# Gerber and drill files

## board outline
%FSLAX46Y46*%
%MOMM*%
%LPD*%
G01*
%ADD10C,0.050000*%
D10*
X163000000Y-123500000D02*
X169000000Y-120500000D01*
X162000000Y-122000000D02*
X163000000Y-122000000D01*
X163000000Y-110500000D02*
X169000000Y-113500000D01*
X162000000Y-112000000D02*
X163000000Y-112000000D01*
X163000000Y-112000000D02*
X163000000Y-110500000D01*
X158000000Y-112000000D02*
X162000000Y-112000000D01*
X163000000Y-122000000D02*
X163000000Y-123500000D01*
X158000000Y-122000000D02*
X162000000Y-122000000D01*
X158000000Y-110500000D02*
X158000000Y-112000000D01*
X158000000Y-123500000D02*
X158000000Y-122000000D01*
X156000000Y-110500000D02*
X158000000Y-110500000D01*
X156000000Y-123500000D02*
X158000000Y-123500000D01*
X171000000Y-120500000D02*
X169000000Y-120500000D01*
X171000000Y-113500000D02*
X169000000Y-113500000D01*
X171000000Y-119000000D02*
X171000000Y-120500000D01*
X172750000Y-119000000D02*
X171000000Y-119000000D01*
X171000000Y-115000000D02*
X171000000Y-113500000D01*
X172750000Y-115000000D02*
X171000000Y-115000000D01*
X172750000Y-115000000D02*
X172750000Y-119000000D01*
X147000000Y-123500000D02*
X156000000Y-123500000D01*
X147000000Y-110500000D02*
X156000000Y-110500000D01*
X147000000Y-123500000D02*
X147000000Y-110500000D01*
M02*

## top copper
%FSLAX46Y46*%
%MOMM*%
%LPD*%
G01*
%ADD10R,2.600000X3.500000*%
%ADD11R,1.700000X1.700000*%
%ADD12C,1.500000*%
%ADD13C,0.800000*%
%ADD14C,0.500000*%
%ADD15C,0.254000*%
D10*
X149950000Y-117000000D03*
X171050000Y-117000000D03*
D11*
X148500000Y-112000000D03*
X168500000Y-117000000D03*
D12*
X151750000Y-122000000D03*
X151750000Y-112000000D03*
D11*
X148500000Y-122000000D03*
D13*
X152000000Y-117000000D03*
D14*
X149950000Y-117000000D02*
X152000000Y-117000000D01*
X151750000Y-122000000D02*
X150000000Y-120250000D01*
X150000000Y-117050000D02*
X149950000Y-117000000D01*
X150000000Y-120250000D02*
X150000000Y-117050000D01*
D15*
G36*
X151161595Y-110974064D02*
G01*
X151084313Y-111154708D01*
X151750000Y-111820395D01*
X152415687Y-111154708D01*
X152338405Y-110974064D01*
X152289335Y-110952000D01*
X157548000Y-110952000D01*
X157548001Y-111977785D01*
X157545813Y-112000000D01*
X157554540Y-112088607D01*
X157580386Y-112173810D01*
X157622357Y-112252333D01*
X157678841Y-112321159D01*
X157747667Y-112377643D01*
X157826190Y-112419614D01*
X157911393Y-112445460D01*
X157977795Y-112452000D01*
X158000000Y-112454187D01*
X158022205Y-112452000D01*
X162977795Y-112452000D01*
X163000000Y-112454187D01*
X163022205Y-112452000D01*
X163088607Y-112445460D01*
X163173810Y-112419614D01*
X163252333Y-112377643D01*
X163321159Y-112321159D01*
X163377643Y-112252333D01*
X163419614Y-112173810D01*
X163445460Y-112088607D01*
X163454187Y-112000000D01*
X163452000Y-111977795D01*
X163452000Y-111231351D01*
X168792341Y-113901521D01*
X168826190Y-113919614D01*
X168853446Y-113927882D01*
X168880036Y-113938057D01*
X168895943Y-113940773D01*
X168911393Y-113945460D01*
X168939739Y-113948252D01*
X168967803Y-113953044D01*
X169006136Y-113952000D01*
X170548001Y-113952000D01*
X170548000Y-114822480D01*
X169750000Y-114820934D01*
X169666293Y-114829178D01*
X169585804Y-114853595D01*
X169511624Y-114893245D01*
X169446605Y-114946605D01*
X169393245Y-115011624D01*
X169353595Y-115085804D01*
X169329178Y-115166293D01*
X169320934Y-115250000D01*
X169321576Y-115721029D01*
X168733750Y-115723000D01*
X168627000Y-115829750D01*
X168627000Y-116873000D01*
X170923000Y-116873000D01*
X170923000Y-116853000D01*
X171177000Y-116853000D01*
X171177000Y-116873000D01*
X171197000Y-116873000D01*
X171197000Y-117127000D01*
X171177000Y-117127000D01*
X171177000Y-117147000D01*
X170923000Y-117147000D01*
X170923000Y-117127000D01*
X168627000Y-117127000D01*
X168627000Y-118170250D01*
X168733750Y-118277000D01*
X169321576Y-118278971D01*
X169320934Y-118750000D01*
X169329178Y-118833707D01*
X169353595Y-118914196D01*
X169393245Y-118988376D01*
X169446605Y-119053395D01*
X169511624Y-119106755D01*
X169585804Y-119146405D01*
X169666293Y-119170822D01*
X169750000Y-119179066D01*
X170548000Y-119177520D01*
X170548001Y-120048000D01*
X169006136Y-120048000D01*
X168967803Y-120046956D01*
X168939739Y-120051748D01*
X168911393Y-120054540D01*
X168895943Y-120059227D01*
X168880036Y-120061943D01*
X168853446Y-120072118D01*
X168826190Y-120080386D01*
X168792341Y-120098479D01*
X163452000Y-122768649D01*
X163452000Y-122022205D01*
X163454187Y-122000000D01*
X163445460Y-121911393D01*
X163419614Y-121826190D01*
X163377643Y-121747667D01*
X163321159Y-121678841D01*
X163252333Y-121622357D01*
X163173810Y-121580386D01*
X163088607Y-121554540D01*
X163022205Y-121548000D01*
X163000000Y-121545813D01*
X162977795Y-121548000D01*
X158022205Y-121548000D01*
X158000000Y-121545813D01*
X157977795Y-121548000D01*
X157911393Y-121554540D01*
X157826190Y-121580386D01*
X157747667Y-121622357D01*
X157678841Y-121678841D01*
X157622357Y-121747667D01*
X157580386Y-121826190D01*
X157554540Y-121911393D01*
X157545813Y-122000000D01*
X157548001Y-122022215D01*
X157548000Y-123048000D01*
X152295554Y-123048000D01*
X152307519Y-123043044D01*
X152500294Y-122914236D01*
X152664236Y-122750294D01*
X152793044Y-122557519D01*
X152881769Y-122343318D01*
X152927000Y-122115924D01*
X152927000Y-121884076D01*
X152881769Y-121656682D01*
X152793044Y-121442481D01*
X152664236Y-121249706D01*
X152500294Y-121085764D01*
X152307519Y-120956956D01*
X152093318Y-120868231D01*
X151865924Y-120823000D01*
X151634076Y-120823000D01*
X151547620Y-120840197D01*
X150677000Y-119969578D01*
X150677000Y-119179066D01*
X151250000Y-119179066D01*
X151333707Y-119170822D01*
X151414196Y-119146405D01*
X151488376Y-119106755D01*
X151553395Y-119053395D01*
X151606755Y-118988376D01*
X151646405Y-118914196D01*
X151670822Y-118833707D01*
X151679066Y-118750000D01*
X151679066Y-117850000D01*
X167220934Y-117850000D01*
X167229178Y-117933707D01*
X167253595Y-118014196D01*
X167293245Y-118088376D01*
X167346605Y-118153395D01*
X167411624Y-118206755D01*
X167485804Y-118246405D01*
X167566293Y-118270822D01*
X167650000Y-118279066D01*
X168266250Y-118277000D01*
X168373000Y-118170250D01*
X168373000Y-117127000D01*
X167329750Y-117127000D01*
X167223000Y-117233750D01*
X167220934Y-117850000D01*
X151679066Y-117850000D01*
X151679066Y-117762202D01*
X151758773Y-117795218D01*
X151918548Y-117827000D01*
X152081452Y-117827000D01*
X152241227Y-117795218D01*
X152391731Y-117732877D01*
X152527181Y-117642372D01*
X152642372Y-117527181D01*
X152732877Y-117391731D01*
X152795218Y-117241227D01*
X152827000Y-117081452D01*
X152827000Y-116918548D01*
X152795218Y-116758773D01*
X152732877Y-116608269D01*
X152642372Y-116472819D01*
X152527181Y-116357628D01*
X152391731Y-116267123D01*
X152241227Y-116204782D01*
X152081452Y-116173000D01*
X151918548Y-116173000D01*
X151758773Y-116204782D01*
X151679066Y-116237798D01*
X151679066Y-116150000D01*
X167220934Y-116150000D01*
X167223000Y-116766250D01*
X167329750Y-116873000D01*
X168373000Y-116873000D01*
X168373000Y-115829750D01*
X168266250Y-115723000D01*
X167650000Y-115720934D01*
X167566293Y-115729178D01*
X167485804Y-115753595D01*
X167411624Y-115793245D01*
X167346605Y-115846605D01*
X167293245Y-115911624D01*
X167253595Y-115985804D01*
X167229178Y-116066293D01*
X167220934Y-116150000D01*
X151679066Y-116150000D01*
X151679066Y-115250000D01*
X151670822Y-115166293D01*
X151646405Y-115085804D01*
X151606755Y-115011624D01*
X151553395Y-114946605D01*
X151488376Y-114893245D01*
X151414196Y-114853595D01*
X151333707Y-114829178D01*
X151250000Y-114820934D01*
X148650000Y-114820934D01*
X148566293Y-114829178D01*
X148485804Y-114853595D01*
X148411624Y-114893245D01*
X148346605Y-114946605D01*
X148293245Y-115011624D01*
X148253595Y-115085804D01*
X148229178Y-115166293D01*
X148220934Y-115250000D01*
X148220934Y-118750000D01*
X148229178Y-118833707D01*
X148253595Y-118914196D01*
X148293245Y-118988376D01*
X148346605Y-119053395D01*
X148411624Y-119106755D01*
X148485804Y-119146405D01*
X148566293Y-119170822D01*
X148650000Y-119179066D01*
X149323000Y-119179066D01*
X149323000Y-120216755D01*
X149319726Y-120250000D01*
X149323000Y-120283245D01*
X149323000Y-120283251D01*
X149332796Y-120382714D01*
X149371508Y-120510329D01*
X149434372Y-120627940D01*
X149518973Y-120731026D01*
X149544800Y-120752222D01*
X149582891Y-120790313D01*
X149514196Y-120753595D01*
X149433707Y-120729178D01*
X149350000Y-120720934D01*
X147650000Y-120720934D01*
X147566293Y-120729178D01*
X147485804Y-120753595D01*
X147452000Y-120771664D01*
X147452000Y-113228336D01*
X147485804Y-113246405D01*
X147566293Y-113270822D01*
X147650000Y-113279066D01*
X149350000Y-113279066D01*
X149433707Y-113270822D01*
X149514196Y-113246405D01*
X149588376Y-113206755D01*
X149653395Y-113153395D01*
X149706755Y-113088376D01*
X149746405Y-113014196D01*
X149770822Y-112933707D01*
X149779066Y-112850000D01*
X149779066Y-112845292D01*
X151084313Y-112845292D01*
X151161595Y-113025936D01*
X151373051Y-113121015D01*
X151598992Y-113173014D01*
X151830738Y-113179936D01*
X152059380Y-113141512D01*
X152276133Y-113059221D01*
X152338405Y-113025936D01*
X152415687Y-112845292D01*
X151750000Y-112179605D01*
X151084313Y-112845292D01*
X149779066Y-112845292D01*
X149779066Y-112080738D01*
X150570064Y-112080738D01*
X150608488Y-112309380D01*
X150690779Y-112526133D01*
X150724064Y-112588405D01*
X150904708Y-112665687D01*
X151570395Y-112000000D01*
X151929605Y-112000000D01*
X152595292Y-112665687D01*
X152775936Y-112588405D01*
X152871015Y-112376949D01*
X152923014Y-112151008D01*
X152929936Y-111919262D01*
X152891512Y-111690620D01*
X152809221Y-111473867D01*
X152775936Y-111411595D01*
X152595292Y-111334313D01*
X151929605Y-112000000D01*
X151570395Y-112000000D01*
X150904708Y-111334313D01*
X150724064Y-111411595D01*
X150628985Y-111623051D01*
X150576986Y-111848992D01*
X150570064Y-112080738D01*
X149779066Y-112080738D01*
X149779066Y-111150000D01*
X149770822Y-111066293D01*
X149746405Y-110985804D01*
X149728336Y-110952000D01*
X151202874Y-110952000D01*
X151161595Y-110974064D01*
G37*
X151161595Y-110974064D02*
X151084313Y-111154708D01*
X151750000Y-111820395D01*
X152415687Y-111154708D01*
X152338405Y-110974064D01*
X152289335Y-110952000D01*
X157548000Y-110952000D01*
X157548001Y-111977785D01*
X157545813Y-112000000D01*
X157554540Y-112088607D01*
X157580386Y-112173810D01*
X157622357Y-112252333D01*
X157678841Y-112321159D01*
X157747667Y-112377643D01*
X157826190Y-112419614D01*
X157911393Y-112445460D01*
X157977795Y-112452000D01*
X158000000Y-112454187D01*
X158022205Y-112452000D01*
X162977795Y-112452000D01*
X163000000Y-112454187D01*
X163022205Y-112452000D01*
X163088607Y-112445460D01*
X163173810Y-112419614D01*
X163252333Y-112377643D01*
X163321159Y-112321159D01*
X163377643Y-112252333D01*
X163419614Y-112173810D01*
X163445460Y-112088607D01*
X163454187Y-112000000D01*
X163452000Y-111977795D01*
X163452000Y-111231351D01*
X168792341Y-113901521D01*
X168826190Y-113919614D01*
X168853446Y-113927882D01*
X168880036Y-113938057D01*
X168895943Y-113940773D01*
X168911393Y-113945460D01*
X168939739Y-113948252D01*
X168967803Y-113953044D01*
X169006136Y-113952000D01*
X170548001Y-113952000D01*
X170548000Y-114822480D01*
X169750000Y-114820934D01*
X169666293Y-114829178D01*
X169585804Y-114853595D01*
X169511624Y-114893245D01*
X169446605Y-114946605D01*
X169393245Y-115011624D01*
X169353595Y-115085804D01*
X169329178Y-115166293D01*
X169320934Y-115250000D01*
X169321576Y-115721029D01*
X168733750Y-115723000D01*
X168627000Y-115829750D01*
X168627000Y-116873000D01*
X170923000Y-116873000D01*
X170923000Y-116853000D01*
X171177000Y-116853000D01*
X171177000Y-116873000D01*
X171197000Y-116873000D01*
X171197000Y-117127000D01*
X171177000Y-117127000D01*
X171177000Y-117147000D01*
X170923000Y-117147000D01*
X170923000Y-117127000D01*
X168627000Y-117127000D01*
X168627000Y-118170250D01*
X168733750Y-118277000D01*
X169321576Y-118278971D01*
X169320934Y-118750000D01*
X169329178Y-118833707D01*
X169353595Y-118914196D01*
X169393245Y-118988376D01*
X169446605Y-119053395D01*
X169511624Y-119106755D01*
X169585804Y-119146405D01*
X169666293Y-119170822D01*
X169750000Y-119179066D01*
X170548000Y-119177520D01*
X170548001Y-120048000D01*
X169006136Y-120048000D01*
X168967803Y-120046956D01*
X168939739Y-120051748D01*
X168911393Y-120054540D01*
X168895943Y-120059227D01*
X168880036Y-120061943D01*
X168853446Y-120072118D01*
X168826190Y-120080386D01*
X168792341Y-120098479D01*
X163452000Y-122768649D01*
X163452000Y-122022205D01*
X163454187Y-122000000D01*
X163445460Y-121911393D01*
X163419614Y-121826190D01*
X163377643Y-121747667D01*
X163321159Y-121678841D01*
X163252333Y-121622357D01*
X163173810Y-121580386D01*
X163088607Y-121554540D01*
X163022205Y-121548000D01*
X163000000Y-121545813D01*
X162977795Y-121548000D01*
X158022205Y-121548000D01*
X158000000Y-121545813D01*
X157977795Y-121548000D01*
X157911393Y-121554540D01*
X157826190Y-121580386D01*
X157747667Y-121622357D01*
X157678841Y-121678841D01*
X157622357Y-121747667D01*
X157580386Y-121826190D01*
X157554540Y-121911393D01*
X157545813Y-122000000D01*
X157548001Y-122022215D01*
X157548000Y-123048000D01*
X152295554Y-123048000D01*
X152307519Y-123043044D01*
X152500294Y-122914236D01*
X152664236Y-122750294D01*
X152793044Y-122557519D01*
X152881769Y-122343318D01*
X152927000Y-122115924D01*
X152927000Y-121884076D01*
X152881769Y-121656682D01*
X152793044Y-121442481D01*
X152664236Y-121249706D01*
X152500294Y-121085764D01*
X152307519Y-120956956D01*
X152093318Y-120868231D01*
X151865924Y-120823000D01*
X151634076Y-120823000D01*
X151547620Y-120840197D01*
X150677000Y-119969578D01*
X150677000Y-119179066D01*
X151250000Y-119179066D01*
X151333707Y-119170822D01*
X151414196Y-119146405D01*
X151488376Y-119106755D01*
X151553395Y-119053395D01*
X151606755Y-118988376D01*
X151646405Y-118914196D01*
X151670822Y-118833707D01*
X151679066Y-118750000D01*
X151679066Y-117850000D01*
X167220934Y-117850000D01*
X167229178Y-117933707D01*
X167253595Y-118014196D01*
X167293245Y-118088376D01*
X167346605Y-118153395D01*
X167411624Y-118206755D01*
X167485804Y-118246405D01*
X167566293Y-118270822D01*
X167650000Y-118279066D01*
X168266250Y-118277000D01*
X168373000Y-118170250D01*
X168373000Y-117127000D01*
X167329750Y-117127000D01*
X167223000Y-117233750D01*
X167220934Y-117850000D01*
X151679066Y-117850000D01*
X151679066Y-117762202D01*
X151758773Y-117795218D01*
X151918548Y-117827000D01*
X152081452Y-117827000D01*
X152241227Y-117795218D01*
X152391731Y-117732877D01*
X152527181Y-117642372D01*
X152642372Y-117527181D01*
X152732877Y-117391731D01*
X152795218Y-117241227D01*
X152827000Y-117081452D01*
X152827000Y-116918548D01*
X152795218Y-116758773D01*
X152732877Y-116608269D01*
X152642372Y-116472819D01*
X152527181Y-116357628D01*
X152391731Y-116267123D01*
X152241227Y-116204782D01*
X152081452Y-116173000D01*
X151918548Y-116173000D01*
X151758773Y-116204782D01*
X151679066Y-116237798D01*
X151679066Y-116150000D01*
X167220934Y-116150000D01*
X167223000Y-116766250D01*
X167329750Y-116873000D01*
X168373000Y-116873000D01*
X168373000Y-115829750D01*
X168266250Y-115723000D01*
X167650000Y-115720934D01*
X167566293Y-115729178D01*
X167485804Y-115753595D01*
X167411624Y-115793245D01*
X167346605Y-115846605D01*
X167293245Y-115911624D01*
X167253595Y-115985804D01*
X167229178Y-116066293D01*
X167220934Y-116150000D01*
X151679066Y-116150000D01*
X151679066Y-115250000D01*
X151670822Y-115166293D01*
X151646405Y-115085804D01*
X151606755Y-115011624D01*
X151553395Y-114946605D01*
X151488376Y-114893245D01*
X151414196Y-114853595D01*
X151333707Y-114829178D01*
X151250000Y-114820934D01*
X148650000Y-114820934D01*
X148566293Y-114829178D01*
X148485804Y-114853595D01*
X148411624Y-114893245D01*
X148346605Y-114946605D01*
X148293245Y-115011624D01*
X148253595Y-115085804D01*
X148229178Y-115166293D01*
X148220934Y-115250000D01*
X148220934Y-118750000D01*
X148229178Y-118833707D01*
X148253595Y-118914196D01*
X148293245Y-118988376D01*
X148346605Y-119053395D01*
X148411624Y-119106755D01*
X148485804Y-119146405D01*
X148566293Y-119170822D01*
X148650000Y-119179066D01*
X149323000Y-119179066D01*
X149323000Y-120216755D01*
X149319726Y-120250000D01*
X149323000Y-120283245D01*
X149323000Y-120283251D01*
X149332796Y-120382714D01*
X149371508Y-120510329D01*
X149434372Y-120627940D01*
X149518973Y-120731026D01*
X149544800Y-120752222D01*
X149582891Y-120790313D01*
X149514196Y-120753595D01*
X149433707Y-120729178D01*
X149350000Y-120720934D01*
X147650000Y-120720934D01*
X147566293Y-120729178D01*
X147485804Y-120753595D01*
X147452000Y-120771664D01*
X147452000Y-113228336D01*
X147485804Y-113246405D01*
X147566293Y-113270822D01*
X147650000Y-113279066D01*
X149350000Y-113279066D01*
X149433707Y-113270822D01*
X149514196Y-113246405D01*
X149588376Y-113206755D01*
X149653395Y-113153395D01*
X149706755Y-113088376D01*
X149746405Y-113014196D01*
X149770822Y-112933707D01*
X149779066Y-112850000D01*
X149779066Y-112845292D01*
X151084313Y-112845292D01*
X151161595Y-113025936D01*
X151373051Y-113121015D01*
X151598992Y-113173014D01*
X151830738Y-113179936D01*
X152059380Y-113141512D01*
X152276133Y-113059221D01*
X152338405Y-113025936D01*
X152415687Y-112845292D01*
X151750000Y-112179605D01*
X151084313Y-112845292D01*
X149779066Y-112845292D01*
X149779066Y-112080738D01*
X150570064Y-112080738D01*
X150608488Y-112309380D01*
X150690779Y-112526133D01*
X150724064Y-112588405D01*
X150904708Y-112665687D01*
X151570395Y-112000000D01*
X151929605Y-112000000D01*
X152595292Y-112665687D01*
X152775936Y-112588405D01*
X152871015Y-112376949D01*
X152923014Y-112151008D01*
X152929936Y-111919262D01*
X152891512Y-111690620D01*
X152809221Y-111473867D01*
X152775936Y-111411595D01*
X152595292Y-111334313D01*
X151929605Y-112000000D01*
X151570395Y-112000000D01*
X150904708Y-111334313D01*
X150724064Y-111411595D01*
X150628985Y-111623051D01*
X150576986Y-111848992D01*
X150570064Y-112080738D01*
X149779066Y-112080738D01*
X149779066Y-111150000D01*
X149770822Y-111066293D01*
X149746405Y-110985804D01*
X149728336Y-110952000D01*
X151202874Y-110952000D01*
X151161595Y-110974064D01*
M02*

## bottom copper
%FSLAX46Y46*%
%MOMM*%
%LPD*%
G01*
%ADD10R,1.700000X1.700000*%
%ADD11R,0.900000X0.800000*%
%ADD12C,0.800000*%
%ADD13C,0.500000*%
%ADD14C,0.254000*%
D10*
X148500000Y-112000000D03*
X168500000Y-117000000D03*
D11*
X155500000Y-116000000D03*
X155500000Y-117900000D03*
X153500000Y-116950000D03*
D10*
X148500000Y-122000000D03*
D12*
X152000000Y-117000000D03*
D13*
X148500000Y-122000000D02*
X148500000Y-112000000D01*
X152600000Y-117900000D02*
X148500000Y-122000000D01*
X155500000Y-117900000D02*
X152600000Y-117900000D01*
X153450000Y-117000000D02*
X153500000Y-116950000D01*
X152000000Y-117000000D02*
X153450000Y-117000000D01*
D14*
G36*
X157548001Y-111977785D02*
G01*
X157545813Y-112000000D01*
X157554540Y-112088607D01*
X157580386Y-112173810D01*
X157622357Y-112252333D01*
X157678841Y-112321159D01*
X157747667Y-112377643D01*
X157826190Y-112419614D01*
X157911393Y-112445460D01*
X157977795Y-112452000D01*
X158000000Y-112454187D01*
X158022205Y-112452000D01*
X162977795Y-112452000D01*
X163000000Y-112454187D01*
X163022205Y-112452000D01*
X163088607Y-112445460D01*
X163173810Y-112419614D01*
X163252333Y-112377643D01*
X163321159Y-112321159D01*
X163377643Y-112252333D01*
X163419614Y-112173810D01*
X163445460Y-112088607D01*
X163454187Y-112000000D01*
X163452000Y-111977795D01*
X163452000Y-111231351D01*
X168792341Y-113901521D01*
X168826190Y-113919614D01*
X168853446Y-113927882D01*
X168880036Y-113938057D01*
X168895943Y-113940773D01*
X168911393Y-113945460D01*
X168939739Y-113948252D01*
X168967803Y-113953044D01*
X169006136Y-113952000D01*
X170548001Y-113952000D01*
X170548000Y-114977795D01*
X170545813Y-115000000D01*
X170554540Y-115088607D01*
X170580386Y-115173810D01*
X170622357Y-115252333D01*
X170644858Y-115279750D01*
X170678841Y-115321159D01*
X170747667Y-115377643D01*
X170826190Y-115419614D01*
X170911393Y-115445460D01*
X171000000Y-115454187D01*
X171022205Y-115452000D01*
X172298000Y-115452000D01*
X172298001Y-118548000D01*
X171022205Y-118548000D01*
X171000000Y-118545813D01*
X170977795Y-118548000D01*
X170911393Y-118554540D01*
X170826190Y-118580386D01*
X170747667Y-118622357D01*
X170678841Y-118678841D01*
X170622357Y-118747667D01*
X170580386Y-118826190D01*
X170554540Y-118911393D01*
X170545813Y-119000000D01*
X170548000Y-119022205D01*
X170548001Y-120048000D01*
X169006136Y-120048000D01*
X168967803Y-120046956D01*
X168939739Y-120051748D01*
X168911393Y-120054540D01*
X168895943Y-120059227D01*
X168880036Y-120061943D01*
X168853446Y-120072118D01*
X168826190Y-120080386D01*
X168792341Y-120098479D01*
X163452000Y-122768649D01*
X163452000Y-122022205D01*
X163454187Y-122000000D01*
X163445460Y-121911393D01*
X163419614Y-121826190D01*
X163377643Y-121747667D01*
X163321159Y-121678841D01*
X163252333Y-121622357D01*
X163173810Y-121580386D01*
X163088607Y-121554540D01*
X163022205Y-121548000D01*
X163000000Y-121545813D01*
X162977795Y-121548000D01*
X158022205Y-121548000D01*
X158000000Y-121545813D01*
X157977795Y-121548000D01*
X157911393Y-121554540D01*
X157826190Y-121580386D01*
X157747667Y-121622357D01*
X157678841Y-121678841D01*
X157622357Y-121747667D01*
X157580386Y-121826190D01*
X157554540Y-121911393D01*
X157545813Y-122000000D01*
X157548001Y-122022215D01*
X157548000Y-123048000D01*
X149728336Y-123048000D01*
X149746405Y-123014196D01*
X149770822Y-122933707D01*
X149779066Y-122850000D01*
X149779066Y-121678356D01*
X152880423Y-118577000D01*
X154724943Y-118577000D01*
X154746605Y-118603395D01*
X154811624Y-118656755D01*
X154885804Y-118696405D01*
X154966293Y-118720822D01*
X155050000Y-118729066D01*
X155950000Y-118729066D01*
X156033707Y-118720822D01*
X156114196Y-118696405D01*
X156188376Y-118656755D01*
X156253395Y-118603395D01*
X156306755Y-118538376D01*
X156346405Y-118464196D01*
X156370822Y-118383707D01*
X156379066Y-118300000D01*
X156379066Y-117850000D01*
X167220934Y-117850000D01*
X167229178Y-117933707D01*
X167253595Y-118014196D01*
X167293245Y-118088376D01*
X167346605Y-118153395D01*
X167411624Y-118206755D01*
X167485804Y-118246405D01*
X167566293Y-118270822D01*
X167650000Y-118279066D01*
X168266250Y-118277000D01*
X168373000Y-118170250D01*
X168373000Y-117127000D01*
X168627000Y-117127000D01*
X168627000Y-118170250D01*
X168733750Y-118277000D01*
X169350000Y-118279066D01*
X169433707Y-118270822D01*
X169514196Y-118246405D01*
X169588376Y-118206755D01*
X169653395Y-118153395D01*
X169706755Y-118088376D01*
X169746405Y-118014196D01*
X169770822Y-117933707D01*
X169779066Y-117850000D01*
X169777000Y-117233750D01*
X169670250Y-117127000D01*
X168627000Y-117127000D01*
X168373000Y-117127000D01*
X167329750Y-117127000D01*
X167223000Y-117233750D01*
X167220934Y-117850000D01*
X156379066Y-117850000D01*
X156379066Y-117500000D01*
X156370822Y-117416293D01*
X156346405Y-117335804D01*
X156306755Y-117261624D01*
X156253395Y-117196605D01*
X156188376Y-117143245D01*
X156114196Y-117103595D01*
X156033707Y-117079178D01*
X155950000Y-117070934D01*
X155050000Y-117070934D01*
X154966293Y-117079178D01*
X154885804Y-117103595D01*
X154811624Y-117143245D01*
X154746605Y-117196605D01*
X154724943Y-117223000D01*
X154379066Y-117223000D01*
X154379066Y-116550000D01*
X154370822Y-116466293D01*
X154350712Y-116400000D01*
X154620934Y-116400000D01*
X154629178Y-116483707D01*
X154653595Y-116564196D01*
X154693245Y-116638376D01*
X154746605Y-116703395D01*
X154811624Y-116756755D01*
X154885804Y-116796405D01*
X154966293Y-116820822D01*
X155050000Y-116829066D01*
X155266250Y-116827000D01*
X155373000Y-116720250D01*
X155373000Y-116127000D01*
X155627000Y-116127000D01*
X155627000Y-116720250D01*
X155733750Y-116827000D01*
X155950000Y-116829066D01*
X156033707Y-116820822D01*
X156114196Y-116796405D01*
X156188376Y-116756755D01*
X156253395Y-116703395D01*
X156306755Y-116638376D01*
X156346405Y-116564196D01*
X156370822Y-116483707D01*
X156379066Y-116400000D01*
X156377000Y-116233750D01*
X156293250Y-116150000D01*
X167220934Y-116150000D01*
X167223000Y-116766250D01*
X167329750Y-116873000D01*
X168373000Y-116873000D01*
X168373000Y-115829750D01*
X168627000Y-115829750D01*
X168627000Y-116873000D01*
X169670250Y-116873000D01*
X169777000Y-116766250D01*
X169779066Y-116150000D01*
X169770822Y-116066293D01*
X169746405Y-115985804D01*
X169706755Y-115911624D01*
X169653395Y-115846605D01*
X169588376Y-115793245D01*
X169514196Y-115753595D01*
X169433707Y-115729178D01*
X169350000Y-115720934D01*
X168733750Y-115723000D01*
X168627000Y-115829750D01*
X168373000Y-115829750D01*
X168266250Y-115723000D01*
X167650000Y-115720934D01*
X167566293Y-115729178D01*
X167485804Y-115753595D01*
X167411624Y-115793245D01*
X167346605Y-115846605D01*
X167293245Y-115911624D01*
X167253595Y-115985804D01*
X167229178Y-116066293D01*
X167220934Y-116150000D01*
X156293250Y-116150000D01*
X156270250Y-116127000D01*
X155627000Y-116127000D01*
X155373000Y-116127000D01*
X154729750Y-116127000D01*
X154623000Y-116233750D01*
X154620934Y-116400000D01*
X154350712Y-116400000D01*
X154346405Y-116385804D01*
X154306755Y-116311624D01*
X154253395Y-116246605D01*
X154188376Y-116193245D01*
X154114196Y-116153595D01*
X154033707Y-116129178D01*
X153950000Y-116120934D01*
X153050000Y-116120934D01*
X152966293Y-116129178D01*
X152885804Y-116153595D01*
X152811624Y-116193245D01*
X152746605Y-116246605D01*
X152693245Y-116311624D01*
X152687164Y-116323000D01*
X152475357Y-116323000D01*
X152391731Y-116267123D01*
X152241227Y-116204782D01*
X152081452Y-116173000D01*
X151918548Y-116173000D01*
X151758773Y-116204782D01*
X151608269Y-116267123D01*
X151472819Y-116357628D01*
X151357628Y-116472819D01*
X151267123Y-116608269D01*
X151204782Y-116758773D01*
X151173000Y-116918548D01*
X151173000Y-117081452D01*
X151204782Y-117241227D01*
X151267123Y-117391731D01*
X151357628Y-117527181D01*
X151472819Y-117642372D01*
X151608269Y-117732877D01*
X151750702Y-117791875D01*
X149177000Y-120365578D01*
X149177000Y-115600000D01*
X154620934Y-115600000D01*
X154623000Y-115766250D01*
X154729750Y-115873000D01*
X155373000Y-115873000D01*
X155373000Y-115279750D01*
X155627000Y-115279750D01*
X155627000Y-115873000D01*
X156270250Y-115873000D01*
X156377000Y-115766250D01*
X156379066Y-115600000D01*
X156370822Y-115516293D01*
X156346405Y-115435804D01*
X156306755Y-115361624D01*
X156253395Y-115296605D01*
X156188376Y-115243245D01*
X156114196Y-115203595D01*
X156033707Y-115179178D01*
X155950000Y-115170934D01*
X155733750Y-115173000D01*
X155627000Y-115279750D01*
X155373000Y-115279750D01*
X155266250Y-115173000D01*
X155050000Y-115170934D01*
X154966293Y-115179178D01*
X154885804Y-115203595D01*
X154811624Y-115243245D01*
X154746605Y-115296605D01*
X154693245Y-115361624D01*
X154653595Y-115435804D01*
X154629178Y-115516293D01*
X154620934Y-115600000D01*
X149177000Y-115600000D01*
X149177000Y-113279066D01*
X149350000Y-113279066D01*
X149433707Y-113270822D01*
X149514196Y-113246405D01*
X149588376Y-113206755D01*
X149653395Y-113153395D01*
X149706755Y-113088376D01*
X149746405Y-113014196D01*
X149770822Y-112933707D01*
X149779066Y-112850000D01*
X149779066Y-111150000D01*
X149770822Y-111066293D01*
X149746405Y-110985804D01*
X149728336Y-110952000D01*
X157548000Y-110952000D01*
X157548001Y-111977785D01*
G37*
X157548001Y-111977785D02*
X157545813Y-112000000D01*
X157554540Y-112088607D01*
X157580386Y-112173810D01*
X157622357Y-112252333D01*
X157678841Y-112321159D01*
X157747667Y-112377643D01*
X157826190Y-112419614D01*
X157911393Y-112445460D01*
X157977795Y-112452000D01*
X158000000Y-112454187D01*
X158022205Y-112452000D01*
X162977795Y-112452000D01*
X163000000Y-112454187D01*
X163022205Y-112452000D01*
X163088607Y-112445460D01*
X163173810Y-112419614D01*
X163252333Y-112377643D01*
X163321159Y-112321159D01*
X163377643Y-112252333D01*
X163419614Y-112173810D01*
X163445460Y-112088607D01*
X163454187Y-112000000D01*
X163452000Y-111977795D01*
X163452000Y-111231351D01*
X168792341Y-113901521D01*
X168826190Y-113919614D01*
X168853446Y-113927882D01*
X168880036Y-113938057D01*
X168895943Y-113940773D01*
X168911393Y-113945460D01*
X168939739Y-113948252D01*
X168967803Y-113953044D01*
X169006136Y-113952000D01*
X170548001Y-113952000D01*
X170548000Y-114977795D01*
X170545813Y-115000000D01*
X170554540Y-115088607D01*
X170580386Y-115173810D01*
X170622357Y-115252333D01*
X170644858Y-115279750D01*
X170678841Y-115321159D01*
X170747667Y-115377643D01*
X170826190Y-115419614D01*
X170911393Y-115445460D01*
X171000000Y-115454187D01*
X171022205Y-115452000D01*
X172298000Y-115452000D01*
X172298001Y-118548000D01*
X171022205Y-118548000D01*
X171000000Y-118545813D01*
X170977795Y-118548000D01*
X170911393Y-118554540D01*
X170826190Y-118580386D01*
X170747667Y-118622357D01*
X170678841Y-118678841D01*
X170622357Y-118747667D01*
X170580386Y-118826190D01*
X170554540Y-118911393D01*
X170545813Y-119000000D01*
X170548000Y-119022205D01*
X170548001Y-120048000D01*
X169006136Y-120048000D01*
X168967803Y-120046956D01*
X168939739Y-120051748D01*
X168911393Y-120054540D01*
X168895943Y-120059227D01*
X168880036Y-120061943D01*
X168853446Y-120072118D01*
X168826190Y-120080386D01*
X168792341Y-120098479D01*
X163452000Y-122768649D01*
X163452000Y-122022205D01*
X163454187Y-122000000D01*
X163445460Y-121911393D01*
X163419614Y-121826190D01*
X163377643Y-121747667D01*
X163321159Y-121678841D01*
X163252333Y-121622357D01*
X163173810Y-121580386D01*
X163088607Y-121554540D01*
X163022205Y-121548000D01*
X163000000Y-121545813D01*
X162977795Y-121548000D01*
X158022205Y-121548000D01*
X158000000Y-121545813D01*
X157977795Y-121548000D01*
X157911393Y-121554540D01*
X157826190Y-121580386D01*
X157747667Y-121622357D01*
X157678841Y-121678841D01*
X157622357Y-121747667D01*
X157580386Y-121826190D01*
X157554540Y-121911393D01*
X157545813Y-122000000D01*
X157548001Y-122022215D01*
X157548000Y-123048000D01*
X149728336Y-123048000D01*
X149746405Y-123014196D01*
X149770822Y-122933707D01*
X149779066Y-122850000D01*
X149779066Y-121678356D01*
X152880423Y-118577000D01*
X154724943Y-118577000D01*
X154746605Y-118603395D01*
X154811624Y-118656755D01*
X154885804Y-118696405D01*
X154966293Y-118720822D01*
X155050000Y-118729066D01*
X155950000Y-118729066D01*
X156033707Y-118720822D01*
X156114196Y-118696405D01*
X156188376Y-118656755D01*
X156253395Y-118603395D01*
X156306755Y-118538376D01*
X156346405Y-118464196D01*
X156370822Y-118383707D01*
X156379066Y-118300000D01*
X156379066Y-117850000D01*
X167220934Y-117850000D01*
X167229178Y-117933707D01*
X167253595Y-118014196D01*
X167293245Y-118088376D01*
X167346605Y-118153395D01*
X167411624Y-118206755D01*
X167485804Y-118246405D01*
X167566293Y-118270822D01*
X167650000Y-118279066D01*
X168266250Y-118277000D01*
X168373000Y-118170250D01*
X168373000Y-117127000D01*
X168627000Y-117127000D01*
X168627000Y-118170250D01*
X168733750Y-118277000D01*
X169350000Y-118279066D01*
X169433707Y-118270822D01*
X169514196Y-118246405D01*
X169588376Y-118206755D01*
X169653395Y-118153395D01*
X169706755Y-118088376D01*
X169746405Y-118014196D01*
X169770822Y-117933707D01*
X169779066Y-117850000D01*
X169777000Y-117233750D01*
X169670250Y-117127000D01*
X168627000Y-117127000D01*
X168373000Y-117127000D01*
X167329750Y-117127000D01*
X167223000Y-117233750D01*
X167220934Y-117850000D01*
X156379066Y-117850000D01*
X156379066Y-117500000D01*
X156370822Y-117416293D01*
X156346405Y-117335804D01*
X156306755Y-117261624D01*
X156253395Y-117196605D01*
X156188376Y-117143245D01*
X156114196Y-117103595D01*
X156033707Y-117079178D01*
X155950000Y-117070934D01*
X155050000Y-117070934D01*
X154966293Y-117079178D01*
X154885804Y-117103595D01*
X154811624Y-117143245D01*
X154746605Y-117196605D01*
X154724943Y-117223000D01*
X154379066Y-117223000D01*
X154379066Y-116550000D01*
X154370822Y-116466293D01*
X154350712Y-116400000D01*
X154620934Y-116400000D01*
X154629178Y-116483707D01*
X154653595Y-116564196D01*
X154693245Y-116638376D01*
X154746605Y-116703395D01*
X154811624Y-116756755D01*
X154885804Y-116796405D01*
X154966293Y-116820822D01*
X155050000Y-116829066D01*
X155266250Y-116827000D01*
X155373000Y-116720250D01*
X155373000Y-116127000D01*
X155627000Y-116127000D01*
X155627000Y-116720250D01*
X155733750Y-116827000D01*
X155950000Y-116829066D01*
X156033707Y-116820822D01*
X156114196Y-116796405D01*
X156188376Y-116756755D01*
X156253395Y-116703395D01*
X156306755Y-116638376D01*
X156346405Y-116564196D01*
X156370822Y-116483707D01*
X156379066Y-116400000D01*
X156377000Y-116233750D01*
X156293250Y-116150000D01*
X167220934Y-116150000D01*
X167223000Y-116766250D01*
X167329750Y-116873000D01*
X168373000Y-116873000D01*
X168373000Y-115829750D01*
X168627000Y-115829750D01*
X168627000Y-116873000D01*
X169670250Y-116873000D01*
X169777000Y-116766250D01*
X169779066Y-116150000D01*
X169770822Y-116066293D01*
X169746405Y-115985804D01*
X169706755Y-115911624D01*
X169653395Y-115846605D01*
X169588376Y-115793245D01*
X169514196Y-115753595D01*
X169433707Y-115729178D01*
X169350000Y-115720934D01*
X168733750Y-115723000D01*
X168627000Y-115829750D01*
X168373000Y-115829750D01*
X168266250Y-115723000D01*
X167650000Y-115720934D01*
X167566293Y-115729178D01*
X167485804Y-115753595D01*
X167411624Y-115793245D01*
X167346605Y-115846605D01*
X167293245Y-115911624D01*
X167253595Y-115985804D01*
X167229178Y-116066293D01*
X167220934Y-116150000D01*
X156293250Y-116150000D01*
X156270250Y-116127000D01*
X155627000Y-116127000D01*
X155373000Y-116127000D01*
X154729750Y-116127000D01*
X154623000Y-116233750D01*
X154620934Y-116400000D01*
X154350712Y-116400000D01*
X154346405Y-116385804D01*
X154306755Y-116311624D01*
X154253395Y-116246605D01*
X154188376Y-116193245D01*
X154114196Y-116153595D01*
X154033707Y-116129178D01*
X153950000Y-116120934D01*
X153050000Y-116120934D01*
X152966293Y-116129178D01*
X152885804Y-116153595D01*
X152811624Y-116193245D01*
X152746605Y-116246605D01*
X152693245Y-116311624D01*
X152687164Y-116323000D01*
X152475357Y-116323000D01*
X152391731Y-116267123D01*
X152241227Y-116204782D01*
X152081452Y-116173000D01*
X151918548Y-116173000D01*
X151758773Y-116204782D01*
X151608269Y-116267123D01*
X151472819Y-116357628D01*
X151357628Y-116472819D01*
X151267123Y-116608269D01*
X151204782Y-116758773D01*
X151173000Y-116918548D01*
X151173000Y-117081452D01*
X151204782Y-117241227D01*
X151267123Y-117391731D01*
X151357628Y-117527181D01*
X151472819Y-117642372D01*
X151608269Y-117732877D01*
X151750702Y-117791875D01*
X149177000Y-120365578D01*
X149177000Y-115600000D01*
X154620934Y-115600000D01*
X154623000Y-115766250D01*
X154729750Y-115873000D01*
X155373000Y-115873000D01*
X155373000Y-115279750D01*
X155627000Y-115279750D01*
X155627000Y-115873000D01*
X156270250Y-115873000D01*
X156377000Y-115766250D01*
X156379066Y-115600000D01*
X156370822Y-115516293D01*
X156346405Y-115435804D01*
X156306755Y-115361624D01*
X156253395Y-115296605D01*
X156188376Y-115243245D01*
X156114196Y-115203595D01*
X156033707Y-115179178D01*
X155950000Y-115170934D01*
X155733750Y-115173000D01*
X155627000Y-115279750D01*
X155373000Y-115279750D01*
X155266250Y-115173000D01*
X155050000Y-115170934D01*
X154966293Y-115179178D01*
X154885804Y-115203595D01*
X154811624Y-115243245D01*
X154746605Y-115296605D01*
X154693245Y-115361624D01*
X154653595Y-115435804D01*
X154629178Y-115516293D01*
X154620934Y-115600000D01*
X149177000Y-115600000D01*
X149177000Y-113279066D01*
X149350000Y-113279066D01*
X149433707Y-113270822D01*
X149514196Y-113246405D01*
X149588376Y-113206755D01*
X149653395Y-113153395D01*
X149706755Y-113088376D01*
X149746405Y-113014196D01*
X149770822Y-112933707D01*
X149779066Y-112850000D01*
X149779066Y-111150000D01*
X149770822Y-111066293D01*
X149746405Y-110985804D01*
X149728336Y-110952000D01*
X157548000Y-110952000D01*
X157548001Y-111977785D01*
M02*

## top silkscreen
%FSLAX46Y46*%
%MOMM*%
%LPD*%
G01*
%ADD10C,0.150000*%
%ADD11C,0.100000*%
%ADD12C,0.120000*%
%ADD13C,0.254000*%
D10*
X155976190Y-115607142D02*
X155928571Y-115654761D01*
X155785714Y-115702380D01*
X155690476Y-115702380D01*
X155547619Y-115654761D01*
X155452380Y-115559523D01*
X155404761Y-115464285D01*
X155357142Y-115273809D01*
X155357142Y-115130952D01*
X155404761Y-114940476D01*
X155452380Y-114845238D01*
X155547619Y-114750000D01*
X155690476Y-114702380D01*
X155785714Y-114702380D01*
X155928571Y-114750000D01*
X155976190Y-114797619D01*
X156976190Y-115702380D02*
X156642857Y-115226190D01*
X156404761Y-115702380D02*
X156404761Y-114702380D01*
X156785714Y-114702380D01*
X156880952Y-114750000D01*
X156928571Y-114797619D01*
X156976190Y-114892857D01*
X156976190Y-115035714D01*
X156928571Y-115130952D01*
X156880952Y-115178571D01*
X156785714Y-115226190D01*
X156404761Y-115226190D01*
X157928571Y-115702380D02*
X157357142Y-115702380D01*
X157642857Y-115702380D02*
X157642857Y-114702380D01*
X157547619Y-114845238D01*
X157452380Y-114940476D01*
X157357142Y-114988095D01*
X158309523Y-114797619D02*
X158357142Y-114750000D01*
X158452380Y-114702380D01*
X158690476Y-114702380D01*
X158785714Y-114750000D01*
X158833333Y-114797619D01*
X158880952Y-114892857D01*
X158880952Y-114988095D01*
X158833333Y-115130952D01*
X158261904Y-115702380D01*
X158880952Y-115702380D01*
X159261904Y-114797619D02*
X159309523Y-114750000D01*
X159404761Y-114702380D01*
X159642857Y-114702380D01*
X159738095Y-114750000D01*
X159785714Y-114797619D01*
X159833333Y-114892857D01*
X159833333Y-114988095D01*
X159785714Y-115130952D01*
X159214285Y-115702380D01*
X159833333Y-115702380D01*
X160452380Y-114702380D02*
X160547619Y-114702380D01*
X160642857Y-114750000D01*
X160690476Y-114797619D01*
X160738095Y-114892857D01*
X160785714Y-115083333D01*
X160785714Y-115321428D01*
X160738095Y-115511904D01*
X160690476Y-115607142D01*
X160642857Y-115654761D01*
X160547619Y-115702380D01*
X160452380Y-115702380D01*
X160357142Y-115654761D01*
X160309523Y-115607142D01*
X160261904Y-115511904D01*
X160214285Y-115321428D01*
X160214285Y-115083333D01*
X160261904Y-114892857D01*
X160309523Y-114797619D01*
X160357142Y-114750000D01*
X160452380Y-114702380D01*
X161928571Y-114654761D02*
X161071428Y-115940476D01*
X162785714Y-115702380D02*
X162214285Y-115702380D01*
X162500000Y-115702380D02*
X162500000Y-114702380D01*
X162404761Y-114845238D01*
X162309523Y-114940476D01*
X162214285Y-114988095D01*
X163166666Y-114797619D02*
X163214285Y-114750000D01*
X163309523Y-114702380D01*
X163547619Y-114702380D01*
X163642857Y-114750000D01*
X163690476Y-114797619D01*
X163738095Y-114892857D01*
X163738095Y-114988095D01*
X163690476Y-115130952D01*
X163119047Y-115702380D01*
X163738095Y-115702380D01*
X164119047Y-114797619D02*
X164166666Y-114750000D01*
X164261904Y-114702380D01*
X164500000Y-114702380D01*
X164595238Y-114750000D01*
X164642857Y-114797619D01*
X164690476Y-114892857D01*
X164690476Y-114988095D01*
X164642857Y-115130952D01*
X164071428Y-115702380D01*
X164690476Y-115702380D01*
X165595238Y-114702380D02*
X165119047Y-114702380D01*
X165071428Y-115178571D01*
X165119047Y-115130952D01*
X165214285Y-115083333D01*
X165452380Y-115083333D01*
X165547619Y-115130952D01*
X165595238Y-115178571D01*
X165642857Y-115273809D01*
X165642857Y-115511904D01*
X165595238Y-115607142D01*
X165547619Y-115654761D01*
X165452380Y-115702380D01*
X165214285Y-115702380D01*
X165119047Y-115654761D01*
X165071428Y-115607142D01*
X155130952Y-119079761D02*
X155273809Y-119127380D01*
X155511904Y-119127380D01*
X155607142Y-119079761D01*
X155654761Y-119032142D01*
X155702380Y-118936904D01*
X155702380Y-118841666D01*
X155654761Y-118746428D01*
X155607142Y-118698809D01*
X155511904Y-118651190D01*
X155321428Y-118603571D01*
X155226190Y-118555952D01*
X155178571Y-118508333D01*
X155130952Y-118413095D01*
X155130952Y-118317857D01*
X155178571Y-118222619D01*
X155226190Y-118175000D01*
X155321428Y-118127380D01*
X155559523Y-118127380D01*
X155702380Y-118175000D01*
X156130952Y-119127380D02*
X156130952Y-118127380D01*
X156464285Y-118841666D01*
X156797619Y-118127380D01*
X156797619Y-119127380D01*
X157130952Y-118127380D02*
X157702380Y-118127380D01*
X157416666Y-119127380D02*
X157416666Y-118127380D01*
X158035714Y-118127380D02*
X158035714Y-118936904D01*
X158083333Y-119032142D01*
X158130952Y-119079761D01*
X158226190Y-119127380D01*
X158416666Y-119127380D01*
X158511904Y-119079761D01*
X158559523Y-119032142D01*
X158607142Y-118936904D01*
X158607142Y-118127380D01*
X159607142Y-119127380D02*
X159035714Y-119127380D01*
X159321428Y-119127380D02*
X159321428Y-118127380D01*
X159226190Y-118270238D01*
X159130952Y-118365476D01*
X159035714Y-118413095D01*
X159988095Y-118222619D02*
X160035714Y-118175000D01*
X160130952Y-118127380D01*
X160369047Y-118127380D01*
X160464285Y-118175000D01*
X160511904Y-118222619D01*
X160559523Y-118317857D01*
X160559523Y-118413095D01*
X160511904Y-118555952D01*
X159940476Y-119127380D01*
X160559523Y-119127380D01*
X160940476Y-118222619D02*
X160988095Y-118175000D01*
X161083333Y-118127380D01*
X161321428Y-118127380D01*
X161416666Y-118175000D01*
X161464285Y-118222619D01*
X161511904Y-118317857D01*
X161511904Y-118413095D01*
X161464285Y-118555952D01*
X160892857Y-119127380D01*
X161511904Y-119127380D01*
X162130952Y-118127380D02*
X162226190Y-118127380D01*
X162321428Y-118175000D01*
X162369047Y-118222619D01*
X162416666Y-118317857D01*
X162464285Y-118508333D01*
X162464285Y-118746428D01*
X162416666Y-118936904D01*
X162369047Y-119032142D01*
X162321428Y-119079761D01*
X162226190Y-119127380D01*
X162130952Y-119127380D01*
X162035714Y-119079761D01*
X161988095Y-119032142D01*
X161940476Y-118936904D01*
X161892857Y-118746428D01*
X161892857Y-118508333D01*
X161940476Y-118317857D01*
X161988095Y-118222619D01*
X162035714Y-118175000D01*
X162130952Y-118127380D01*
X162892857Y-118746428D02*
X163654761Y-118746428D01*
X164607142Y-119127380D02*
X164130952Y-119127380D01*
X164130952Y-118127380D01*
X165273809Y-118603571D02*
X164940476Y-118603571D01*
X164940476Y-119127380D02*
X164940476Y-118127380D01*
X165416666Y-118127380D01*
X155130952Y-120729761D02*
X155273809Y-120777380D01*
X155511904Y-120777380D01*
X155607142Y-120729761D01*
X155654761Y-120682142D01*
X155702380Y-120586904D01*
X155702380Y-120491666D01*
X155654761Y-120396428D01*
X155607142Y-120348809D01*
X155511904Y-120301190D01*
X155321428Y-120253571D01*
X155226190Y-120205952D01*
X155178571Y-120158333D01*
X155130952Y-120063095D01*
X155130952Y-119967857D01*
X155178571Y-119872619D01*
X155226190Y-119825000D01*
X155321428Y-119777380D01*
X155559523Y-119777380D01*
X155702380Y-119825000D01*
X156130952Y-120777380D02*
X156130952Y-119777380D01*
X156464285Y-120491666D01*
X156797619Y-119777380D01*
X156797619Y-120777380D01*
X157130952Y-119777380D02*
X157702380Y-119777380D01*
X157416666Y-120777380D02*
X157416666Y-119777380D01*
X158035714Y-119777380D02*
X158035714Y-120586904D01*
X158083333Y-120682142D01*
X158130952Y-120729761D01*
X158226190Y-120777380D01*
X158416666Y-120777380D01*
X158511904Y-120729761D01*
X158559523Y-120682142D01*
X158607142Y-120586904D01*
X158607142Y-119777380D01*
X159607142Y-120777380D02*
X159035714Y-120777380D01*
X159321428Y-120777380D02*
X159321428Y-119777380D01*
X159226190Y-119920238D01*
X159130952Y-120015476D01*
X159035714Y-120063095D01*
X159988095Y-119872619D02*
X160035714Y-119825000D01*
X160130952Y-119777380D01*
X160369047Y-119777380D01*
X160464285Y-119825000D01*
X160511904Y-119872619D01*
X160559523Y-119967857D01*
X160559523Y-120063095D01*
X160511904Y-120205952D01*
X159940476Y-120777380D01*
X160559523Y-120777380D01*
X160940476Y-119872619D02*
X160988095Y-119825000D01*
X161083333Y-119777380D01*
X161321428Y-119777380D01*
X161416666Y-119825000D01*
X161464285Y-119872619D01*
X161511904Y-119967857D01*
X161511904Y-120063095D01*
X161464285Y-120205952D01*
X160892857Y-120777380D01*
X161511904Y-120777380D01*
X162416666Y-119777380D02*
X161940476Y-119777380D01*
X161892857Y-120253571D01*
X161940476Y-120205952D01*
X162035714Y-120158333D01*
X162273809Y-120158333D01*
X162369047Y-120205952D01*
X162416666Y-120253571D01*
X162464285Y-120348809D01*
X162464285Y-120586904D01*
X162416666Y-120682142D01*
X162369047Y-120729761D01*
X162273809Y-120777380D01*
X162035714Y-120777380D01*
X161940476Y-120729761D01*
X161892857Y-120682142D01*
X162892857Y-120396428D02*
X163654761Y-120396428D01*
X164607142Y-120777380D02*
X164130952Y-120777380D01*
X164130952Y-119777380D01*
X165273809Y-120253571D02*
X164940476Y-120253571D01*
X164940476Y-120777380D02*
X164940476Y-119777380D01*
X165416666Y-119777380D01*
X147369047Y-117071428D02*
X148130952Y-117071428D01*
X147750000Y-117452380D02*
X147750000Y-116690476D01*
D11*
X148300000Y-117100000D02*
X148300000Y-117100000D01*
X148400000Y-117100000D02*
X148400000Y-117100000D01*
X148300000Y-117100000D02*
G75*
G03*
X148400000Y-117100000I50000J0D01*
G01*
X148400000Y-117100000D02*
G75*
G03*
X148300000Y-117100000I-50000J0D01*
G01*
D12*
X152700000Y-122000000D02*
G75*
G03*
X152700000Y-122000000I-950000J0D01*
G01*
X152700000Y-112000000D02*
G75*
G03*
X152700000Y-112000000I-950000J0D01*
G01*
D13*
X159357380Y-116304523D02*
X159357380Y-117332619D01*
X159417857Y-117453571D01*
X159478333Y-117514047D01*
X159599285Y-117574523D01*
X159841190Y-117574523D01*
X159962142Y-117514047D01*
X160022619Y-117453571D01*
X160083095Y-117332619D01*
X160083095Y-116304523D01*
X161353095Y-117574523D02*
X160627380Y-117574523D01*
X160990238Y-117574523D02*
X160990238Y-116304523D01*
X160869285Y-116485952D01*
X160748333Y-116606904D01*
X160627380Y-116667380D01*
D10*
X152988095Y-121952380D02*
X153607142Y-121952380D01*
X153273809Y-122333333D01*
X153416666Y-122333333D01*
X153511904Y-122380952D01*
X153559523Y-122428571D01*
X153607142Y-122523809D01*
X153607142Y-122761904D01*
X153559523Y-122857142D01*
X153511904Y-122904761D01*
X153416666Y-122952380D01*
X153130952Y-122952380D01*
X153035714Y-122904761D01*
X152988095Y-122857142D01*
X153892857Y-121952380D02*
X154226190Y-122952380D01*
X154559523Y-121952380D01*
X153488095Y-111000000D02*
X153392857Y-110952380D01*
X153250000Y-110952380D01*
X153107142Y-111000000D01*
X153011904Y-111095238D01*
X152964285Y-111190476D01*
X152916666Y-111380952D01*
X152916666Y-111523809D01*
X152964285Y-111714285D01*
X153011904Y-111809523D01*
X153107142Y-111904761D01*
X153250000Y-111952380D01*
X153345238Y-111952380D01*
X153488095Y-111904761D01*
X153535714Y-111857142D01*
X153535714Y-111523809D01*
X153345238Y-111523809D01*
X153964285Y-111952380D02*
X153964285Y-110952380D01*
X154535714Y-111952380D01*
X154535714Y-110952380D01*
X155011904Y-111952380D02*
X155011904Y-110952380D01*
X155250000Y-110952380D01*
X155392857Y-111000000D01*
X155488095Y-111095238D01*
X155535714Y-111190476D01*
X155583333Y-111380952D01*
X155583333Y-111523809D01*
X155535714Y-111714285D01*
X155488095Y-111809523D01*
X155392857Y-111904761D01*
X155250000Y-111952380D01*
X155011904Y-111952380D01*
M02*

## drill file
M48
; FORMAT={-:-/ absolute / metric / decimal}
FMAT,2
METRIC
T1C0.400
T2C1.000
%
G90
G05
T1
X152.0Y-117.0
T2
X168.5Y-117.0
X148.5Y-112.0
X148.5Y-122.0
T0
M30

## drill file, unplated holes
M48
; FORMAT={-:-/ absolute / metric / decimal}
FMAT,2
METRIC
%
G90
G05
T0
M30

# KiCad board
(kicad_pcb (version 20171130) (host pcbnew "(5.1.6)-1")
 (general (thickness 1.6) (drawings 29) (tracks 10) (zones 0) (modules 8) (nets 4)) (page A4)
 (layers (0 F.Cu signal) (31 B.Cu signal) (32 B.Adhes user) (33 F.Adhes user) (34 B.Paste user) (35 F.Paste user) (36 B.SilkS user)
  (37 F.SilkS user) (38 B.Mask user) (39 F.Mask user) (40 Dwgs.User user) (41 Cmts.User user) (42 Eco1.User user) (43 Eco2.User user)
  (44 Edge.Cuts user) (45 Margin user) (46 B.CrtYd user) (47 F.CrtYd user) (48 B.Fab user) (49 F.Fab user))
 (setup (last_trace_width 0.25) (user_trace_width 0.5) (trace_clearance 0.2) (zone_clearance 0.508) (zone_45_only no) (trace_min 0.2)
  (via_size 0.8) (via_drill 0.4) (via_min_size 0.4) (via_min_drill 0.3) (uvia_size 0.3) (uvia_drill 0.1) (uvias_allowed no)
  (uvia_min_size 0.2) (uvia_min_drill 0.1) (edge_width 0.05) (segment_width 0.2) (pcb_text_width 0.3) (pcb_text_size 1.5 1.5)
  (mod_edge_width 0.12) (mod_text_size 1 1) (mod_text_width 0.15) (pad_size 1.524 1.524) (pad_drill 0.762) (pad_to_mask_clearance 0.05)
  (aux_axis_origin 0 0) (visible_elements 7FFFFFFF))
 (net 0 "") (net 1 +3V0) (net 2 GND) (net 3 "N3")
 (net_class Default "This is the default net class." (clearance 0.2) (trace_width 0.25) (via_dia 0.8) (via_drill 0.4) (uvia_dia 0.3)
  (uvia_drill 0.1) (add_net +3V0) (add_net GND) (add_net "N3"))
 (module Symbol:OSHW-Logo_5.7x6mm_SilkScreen (layer B.Cu) (at 150.25 117 180)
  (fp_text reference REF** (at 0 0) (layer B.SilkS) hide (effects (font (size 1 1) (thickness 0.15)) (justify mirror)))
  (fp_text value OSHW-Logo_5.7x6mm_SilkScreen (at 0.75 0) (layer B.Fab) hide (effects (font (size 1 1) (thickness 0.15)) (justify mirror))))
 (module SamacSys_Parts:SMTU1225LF (layer F.Cu) (at 160.5 117)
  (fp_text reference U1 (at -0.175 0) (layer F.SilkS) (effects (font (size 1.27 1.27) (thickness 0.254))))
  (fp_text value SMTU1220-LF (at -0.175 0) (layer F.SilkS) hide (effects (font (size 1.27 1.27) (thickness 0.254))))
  (fp_line (start -12.2 0.1) (end -12.2 0.1) (layer F.SilkS) (width 0.1))
  (fp_line (start -12.1 0.1) (end -12.1 0.1) (layer F.SilkS) (width 0.1))
  (fp_arc (start -12.15 0.1) (end -12.1 0.1) (angle 180) (layer F.SilkS) (width 0.1))
  (fp_arc (start -12.15 0.1) (end -12.2 0.1) (angle 180) (layer F.SilkS) (width 0.1))
  (pad 1 smd rect (at -10.55 0) (size 2.6 3.5) (layers F.Cu F.Paste F.Mask) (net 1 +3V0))
  (pad 2 smd rect (at 10.55 0) (size 2.6 3.5) (layers F.Cu F.Paste F.Mask) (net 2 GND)))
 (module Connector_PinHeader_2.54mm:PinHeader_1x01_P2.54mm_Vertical (layer B.Cu) (at 148.5 112)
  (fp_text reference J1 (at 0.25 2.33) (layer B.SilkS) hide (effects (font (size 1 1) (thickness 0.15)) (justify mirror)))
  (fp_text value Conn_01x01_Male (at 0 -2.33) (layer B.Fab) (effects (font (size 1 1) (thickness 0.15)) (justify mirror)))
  (pad 1 thru_hole rect (at 0 0) (size 1.7 1.7) (drill 1) (layers *.Cu *.Mask) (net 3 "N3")))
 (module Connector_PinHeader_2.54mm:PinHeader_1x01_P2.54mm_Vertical (layer B.Cu) (at 168.5 117)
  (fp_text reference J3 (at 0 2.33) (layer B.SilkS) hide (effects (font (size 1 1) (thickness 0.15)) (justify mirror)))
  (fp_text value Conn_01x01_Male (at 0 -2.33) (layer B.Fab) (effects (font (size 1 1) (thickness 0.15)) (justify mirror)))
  (pad 1 thru_hole rect (at 0 0) (size 1.7 1.7) (drill 1) (layers *.Cu *.Mask) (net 2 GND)))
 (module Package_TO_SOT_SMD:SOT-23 (layer B.Cu) (at 154.5 116.95 180)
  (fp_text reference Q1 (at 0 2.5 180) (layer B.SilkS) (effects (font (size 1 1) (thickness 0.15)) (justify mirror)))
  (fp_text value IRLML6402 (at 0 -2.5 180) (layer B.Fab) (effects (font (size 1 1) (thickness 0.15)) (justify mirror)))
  (pad 1 smd rect (at -1 0.95 180) (size 0.9 0.8) (layers B.Cu B.Paste B.Mask) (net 2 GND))
  (pad 2 smd rect (at -1 -0.95 180) (size 0.9 0.8) (layers B.Cu B.Paste B.Mask) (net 3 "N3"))
  (pad 3 smd rect (at 1 0 180) (size 0.9 0.8) (layers B.Cu B.Paste B.Mask) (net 1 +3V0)))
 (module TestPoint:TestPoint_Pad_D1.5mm (layer F.Cu) (at 151.75 122)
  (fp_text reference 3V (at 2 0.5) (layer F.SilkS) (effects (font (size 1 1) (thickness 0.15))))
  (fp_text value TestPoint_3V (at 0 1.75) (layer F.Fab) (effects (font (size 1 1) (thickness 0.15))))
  (fp_circle (center 0 0) (end 0 0.95) (layer F.SilkS) (width 0.12))
  (pad 1 smd circle (at 0 0) (size 1.5 1.5) (layers F.Cu F.Mask) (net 1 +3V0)))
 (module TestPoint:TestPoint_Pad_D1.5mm (layer F.Cu) (at 151.75 112)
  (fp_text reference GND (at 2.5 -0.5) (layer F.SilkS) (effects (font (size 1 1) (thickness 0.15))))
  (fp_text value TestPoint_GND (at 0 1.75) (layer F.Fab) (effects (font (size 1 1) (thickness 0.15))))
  (fp_circle (center 0 0) (end 0 0.95) (layer F.SilkS) (width 0.12))
  (pad 1 smd circle (at 0 0) (size 1.5 1.5) (layers F.Cu F.Mask) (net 2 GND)))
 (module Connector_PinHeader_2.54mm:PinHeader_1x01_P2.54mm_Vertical (layer B.Cu) (at 148.5 122)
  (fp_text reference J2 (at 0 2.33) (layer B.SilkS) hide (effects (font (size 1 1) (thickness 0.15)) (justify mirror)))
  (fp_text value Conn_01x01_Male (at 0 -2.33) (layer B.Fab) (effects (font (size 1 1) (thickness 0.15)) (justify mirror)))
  (pad 1 thru_hole rect (at 0 0) (size 1.7 1.7) (drill 1) (layers *.Cu *.Mask) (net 3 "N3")))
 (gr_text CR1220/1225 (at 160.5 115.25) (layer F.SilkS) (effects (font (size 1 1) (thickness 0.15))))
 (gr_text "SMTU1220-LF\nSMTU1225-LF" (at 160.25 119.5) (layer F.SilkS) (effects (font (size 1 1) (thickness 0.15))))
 (gr_line (start 163 123.5) (end 169 120.5) (layer Edge.Cuts) (width 0.05))
 (gr_line (start 162 122) (end 163 122) (layer Edge.Cuts) (width 0.05))
 (gr_line (start 163 110.5) (end 169 113.5) (layer Edge.Cuts) (width 0.05))
 (gr_line (start 162 112) (end 163 112) (layer Edge.Cuts) (width 0.05))
 (gr_line (start 163 112) (end 163 110.5) (layer Edge.Cuts) (width 0.05))
 (gr_line (start 158 112) (end 162 112) (layer Edge.Cuts) (width 0.05))
 (gr_line (start 163 122) (end 163 123.5) (layer Edge.Cuts) (width 0.05))
 (gr_line (start 158 122) (end 162 122) (layer Edge.Cuts) (width 0.05))
 (gr_line (start 158 110.5) (end 158 112) (layer Edge.Cuts) (width 0.05))
 (gr_line (start 158 123.5) (end 158 122) (layer Edge.Cuts) (width 0.05))
 (gr_line (start 156 110.5) (end 158 110.5) (layer Edge.Cuts) (width 0.05))
 (gr_line (start 156 123.5) (end 158 123.5) (layer Edge.Cuts) (width 0.05))
 (gr_line (start 171 120.5) (end 169 120.5) (layer Edge.Cuts) (width 0.05))
 (gr_line (start 171 113.5) (end 169 113.5) (layer Edge.Cuts) (width 0.05))
 (gr_line (start 171 119) (end 171 120.5) (layer Edge.Cuts) (width 0.05))
 (gr_line (start 172.75 119) (end 171 119) (layer Edge.Cuts) (width 0.05))
 (gr_line (start 171 115) (end 171 113.5) (layer Edge.Cuts) (width 0.05))
 (gr_line (start 172.75 115) (end 171 115) (layer Edge.Cuts) (width 0.05))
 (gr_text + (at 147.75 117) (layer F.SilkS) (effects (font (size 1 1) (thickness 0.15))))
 (gr_line (start 172.75 115) (end 172.75 119) (layer Edge.Cuts) (width 0.05))
 (gr_line (start 147 123.5) (end 156 123.5) (layer Edge.Cuts) (width 0.05))
 (gr_line (start 147 110.5) (end 156 110.5) (layer Edge.Cuts) (width 0.05))
 (gr_line (start 147 123.5) (end 147 110.5) (layer Edge.Cuts) (width 0.05))
 (segment (start 148.5 122) (end 148.5 112) (width 0.5) (layer B.Cu) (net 3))
 (segment (start 152.6 117.9) (end 148.5 122) (width 0.5) (layer B.Cu) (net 3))
 (segment (start 155.5 117.9) (end 152.6 117.9) (width 0.5) (layer B.Cu) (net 3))
 (via (at 152 117) (size 0.8) (drill 0.4) (layers F.Cu B.Cu) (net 1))
 (segment (start 149.95 117) (end 152 117) (width 0.5) (layer F.Cu) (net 1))
 (segment (start 153.45 117) (end 153.5 116.95) (width 0.5) (layer B.Cu) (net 1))
 (segment (start 152 117) (end 153.45 117) (width 0.5) (layer B.Cu) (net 1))
 (segment (start 151.75 122) (end 150 120.25) (width 0.5) (layer F.Cu) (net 1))
 (segment (start 150 117.05) (end 149.95 117) (width 0.5) (layer F.Cu) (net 1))
 (segment (start 150 120.25) (end 150 117.05) (width 0.5) (layer F.Cu) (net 1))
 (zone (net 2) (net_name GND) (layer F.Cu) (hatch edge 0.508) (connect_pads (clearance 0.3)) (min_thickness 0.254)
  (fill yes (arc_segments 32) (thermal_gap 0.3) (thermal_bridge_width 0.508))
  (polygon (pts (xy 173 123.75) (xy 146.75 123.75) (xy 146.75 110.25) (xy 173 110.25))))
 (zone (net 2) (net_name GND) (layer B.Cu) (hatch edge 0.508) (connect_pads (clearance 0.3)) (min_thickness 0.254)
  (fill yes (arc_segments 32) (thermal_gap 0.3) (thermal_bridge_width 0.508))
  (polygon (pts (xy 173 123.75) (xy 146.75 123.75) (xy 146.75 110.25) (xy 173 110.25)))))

